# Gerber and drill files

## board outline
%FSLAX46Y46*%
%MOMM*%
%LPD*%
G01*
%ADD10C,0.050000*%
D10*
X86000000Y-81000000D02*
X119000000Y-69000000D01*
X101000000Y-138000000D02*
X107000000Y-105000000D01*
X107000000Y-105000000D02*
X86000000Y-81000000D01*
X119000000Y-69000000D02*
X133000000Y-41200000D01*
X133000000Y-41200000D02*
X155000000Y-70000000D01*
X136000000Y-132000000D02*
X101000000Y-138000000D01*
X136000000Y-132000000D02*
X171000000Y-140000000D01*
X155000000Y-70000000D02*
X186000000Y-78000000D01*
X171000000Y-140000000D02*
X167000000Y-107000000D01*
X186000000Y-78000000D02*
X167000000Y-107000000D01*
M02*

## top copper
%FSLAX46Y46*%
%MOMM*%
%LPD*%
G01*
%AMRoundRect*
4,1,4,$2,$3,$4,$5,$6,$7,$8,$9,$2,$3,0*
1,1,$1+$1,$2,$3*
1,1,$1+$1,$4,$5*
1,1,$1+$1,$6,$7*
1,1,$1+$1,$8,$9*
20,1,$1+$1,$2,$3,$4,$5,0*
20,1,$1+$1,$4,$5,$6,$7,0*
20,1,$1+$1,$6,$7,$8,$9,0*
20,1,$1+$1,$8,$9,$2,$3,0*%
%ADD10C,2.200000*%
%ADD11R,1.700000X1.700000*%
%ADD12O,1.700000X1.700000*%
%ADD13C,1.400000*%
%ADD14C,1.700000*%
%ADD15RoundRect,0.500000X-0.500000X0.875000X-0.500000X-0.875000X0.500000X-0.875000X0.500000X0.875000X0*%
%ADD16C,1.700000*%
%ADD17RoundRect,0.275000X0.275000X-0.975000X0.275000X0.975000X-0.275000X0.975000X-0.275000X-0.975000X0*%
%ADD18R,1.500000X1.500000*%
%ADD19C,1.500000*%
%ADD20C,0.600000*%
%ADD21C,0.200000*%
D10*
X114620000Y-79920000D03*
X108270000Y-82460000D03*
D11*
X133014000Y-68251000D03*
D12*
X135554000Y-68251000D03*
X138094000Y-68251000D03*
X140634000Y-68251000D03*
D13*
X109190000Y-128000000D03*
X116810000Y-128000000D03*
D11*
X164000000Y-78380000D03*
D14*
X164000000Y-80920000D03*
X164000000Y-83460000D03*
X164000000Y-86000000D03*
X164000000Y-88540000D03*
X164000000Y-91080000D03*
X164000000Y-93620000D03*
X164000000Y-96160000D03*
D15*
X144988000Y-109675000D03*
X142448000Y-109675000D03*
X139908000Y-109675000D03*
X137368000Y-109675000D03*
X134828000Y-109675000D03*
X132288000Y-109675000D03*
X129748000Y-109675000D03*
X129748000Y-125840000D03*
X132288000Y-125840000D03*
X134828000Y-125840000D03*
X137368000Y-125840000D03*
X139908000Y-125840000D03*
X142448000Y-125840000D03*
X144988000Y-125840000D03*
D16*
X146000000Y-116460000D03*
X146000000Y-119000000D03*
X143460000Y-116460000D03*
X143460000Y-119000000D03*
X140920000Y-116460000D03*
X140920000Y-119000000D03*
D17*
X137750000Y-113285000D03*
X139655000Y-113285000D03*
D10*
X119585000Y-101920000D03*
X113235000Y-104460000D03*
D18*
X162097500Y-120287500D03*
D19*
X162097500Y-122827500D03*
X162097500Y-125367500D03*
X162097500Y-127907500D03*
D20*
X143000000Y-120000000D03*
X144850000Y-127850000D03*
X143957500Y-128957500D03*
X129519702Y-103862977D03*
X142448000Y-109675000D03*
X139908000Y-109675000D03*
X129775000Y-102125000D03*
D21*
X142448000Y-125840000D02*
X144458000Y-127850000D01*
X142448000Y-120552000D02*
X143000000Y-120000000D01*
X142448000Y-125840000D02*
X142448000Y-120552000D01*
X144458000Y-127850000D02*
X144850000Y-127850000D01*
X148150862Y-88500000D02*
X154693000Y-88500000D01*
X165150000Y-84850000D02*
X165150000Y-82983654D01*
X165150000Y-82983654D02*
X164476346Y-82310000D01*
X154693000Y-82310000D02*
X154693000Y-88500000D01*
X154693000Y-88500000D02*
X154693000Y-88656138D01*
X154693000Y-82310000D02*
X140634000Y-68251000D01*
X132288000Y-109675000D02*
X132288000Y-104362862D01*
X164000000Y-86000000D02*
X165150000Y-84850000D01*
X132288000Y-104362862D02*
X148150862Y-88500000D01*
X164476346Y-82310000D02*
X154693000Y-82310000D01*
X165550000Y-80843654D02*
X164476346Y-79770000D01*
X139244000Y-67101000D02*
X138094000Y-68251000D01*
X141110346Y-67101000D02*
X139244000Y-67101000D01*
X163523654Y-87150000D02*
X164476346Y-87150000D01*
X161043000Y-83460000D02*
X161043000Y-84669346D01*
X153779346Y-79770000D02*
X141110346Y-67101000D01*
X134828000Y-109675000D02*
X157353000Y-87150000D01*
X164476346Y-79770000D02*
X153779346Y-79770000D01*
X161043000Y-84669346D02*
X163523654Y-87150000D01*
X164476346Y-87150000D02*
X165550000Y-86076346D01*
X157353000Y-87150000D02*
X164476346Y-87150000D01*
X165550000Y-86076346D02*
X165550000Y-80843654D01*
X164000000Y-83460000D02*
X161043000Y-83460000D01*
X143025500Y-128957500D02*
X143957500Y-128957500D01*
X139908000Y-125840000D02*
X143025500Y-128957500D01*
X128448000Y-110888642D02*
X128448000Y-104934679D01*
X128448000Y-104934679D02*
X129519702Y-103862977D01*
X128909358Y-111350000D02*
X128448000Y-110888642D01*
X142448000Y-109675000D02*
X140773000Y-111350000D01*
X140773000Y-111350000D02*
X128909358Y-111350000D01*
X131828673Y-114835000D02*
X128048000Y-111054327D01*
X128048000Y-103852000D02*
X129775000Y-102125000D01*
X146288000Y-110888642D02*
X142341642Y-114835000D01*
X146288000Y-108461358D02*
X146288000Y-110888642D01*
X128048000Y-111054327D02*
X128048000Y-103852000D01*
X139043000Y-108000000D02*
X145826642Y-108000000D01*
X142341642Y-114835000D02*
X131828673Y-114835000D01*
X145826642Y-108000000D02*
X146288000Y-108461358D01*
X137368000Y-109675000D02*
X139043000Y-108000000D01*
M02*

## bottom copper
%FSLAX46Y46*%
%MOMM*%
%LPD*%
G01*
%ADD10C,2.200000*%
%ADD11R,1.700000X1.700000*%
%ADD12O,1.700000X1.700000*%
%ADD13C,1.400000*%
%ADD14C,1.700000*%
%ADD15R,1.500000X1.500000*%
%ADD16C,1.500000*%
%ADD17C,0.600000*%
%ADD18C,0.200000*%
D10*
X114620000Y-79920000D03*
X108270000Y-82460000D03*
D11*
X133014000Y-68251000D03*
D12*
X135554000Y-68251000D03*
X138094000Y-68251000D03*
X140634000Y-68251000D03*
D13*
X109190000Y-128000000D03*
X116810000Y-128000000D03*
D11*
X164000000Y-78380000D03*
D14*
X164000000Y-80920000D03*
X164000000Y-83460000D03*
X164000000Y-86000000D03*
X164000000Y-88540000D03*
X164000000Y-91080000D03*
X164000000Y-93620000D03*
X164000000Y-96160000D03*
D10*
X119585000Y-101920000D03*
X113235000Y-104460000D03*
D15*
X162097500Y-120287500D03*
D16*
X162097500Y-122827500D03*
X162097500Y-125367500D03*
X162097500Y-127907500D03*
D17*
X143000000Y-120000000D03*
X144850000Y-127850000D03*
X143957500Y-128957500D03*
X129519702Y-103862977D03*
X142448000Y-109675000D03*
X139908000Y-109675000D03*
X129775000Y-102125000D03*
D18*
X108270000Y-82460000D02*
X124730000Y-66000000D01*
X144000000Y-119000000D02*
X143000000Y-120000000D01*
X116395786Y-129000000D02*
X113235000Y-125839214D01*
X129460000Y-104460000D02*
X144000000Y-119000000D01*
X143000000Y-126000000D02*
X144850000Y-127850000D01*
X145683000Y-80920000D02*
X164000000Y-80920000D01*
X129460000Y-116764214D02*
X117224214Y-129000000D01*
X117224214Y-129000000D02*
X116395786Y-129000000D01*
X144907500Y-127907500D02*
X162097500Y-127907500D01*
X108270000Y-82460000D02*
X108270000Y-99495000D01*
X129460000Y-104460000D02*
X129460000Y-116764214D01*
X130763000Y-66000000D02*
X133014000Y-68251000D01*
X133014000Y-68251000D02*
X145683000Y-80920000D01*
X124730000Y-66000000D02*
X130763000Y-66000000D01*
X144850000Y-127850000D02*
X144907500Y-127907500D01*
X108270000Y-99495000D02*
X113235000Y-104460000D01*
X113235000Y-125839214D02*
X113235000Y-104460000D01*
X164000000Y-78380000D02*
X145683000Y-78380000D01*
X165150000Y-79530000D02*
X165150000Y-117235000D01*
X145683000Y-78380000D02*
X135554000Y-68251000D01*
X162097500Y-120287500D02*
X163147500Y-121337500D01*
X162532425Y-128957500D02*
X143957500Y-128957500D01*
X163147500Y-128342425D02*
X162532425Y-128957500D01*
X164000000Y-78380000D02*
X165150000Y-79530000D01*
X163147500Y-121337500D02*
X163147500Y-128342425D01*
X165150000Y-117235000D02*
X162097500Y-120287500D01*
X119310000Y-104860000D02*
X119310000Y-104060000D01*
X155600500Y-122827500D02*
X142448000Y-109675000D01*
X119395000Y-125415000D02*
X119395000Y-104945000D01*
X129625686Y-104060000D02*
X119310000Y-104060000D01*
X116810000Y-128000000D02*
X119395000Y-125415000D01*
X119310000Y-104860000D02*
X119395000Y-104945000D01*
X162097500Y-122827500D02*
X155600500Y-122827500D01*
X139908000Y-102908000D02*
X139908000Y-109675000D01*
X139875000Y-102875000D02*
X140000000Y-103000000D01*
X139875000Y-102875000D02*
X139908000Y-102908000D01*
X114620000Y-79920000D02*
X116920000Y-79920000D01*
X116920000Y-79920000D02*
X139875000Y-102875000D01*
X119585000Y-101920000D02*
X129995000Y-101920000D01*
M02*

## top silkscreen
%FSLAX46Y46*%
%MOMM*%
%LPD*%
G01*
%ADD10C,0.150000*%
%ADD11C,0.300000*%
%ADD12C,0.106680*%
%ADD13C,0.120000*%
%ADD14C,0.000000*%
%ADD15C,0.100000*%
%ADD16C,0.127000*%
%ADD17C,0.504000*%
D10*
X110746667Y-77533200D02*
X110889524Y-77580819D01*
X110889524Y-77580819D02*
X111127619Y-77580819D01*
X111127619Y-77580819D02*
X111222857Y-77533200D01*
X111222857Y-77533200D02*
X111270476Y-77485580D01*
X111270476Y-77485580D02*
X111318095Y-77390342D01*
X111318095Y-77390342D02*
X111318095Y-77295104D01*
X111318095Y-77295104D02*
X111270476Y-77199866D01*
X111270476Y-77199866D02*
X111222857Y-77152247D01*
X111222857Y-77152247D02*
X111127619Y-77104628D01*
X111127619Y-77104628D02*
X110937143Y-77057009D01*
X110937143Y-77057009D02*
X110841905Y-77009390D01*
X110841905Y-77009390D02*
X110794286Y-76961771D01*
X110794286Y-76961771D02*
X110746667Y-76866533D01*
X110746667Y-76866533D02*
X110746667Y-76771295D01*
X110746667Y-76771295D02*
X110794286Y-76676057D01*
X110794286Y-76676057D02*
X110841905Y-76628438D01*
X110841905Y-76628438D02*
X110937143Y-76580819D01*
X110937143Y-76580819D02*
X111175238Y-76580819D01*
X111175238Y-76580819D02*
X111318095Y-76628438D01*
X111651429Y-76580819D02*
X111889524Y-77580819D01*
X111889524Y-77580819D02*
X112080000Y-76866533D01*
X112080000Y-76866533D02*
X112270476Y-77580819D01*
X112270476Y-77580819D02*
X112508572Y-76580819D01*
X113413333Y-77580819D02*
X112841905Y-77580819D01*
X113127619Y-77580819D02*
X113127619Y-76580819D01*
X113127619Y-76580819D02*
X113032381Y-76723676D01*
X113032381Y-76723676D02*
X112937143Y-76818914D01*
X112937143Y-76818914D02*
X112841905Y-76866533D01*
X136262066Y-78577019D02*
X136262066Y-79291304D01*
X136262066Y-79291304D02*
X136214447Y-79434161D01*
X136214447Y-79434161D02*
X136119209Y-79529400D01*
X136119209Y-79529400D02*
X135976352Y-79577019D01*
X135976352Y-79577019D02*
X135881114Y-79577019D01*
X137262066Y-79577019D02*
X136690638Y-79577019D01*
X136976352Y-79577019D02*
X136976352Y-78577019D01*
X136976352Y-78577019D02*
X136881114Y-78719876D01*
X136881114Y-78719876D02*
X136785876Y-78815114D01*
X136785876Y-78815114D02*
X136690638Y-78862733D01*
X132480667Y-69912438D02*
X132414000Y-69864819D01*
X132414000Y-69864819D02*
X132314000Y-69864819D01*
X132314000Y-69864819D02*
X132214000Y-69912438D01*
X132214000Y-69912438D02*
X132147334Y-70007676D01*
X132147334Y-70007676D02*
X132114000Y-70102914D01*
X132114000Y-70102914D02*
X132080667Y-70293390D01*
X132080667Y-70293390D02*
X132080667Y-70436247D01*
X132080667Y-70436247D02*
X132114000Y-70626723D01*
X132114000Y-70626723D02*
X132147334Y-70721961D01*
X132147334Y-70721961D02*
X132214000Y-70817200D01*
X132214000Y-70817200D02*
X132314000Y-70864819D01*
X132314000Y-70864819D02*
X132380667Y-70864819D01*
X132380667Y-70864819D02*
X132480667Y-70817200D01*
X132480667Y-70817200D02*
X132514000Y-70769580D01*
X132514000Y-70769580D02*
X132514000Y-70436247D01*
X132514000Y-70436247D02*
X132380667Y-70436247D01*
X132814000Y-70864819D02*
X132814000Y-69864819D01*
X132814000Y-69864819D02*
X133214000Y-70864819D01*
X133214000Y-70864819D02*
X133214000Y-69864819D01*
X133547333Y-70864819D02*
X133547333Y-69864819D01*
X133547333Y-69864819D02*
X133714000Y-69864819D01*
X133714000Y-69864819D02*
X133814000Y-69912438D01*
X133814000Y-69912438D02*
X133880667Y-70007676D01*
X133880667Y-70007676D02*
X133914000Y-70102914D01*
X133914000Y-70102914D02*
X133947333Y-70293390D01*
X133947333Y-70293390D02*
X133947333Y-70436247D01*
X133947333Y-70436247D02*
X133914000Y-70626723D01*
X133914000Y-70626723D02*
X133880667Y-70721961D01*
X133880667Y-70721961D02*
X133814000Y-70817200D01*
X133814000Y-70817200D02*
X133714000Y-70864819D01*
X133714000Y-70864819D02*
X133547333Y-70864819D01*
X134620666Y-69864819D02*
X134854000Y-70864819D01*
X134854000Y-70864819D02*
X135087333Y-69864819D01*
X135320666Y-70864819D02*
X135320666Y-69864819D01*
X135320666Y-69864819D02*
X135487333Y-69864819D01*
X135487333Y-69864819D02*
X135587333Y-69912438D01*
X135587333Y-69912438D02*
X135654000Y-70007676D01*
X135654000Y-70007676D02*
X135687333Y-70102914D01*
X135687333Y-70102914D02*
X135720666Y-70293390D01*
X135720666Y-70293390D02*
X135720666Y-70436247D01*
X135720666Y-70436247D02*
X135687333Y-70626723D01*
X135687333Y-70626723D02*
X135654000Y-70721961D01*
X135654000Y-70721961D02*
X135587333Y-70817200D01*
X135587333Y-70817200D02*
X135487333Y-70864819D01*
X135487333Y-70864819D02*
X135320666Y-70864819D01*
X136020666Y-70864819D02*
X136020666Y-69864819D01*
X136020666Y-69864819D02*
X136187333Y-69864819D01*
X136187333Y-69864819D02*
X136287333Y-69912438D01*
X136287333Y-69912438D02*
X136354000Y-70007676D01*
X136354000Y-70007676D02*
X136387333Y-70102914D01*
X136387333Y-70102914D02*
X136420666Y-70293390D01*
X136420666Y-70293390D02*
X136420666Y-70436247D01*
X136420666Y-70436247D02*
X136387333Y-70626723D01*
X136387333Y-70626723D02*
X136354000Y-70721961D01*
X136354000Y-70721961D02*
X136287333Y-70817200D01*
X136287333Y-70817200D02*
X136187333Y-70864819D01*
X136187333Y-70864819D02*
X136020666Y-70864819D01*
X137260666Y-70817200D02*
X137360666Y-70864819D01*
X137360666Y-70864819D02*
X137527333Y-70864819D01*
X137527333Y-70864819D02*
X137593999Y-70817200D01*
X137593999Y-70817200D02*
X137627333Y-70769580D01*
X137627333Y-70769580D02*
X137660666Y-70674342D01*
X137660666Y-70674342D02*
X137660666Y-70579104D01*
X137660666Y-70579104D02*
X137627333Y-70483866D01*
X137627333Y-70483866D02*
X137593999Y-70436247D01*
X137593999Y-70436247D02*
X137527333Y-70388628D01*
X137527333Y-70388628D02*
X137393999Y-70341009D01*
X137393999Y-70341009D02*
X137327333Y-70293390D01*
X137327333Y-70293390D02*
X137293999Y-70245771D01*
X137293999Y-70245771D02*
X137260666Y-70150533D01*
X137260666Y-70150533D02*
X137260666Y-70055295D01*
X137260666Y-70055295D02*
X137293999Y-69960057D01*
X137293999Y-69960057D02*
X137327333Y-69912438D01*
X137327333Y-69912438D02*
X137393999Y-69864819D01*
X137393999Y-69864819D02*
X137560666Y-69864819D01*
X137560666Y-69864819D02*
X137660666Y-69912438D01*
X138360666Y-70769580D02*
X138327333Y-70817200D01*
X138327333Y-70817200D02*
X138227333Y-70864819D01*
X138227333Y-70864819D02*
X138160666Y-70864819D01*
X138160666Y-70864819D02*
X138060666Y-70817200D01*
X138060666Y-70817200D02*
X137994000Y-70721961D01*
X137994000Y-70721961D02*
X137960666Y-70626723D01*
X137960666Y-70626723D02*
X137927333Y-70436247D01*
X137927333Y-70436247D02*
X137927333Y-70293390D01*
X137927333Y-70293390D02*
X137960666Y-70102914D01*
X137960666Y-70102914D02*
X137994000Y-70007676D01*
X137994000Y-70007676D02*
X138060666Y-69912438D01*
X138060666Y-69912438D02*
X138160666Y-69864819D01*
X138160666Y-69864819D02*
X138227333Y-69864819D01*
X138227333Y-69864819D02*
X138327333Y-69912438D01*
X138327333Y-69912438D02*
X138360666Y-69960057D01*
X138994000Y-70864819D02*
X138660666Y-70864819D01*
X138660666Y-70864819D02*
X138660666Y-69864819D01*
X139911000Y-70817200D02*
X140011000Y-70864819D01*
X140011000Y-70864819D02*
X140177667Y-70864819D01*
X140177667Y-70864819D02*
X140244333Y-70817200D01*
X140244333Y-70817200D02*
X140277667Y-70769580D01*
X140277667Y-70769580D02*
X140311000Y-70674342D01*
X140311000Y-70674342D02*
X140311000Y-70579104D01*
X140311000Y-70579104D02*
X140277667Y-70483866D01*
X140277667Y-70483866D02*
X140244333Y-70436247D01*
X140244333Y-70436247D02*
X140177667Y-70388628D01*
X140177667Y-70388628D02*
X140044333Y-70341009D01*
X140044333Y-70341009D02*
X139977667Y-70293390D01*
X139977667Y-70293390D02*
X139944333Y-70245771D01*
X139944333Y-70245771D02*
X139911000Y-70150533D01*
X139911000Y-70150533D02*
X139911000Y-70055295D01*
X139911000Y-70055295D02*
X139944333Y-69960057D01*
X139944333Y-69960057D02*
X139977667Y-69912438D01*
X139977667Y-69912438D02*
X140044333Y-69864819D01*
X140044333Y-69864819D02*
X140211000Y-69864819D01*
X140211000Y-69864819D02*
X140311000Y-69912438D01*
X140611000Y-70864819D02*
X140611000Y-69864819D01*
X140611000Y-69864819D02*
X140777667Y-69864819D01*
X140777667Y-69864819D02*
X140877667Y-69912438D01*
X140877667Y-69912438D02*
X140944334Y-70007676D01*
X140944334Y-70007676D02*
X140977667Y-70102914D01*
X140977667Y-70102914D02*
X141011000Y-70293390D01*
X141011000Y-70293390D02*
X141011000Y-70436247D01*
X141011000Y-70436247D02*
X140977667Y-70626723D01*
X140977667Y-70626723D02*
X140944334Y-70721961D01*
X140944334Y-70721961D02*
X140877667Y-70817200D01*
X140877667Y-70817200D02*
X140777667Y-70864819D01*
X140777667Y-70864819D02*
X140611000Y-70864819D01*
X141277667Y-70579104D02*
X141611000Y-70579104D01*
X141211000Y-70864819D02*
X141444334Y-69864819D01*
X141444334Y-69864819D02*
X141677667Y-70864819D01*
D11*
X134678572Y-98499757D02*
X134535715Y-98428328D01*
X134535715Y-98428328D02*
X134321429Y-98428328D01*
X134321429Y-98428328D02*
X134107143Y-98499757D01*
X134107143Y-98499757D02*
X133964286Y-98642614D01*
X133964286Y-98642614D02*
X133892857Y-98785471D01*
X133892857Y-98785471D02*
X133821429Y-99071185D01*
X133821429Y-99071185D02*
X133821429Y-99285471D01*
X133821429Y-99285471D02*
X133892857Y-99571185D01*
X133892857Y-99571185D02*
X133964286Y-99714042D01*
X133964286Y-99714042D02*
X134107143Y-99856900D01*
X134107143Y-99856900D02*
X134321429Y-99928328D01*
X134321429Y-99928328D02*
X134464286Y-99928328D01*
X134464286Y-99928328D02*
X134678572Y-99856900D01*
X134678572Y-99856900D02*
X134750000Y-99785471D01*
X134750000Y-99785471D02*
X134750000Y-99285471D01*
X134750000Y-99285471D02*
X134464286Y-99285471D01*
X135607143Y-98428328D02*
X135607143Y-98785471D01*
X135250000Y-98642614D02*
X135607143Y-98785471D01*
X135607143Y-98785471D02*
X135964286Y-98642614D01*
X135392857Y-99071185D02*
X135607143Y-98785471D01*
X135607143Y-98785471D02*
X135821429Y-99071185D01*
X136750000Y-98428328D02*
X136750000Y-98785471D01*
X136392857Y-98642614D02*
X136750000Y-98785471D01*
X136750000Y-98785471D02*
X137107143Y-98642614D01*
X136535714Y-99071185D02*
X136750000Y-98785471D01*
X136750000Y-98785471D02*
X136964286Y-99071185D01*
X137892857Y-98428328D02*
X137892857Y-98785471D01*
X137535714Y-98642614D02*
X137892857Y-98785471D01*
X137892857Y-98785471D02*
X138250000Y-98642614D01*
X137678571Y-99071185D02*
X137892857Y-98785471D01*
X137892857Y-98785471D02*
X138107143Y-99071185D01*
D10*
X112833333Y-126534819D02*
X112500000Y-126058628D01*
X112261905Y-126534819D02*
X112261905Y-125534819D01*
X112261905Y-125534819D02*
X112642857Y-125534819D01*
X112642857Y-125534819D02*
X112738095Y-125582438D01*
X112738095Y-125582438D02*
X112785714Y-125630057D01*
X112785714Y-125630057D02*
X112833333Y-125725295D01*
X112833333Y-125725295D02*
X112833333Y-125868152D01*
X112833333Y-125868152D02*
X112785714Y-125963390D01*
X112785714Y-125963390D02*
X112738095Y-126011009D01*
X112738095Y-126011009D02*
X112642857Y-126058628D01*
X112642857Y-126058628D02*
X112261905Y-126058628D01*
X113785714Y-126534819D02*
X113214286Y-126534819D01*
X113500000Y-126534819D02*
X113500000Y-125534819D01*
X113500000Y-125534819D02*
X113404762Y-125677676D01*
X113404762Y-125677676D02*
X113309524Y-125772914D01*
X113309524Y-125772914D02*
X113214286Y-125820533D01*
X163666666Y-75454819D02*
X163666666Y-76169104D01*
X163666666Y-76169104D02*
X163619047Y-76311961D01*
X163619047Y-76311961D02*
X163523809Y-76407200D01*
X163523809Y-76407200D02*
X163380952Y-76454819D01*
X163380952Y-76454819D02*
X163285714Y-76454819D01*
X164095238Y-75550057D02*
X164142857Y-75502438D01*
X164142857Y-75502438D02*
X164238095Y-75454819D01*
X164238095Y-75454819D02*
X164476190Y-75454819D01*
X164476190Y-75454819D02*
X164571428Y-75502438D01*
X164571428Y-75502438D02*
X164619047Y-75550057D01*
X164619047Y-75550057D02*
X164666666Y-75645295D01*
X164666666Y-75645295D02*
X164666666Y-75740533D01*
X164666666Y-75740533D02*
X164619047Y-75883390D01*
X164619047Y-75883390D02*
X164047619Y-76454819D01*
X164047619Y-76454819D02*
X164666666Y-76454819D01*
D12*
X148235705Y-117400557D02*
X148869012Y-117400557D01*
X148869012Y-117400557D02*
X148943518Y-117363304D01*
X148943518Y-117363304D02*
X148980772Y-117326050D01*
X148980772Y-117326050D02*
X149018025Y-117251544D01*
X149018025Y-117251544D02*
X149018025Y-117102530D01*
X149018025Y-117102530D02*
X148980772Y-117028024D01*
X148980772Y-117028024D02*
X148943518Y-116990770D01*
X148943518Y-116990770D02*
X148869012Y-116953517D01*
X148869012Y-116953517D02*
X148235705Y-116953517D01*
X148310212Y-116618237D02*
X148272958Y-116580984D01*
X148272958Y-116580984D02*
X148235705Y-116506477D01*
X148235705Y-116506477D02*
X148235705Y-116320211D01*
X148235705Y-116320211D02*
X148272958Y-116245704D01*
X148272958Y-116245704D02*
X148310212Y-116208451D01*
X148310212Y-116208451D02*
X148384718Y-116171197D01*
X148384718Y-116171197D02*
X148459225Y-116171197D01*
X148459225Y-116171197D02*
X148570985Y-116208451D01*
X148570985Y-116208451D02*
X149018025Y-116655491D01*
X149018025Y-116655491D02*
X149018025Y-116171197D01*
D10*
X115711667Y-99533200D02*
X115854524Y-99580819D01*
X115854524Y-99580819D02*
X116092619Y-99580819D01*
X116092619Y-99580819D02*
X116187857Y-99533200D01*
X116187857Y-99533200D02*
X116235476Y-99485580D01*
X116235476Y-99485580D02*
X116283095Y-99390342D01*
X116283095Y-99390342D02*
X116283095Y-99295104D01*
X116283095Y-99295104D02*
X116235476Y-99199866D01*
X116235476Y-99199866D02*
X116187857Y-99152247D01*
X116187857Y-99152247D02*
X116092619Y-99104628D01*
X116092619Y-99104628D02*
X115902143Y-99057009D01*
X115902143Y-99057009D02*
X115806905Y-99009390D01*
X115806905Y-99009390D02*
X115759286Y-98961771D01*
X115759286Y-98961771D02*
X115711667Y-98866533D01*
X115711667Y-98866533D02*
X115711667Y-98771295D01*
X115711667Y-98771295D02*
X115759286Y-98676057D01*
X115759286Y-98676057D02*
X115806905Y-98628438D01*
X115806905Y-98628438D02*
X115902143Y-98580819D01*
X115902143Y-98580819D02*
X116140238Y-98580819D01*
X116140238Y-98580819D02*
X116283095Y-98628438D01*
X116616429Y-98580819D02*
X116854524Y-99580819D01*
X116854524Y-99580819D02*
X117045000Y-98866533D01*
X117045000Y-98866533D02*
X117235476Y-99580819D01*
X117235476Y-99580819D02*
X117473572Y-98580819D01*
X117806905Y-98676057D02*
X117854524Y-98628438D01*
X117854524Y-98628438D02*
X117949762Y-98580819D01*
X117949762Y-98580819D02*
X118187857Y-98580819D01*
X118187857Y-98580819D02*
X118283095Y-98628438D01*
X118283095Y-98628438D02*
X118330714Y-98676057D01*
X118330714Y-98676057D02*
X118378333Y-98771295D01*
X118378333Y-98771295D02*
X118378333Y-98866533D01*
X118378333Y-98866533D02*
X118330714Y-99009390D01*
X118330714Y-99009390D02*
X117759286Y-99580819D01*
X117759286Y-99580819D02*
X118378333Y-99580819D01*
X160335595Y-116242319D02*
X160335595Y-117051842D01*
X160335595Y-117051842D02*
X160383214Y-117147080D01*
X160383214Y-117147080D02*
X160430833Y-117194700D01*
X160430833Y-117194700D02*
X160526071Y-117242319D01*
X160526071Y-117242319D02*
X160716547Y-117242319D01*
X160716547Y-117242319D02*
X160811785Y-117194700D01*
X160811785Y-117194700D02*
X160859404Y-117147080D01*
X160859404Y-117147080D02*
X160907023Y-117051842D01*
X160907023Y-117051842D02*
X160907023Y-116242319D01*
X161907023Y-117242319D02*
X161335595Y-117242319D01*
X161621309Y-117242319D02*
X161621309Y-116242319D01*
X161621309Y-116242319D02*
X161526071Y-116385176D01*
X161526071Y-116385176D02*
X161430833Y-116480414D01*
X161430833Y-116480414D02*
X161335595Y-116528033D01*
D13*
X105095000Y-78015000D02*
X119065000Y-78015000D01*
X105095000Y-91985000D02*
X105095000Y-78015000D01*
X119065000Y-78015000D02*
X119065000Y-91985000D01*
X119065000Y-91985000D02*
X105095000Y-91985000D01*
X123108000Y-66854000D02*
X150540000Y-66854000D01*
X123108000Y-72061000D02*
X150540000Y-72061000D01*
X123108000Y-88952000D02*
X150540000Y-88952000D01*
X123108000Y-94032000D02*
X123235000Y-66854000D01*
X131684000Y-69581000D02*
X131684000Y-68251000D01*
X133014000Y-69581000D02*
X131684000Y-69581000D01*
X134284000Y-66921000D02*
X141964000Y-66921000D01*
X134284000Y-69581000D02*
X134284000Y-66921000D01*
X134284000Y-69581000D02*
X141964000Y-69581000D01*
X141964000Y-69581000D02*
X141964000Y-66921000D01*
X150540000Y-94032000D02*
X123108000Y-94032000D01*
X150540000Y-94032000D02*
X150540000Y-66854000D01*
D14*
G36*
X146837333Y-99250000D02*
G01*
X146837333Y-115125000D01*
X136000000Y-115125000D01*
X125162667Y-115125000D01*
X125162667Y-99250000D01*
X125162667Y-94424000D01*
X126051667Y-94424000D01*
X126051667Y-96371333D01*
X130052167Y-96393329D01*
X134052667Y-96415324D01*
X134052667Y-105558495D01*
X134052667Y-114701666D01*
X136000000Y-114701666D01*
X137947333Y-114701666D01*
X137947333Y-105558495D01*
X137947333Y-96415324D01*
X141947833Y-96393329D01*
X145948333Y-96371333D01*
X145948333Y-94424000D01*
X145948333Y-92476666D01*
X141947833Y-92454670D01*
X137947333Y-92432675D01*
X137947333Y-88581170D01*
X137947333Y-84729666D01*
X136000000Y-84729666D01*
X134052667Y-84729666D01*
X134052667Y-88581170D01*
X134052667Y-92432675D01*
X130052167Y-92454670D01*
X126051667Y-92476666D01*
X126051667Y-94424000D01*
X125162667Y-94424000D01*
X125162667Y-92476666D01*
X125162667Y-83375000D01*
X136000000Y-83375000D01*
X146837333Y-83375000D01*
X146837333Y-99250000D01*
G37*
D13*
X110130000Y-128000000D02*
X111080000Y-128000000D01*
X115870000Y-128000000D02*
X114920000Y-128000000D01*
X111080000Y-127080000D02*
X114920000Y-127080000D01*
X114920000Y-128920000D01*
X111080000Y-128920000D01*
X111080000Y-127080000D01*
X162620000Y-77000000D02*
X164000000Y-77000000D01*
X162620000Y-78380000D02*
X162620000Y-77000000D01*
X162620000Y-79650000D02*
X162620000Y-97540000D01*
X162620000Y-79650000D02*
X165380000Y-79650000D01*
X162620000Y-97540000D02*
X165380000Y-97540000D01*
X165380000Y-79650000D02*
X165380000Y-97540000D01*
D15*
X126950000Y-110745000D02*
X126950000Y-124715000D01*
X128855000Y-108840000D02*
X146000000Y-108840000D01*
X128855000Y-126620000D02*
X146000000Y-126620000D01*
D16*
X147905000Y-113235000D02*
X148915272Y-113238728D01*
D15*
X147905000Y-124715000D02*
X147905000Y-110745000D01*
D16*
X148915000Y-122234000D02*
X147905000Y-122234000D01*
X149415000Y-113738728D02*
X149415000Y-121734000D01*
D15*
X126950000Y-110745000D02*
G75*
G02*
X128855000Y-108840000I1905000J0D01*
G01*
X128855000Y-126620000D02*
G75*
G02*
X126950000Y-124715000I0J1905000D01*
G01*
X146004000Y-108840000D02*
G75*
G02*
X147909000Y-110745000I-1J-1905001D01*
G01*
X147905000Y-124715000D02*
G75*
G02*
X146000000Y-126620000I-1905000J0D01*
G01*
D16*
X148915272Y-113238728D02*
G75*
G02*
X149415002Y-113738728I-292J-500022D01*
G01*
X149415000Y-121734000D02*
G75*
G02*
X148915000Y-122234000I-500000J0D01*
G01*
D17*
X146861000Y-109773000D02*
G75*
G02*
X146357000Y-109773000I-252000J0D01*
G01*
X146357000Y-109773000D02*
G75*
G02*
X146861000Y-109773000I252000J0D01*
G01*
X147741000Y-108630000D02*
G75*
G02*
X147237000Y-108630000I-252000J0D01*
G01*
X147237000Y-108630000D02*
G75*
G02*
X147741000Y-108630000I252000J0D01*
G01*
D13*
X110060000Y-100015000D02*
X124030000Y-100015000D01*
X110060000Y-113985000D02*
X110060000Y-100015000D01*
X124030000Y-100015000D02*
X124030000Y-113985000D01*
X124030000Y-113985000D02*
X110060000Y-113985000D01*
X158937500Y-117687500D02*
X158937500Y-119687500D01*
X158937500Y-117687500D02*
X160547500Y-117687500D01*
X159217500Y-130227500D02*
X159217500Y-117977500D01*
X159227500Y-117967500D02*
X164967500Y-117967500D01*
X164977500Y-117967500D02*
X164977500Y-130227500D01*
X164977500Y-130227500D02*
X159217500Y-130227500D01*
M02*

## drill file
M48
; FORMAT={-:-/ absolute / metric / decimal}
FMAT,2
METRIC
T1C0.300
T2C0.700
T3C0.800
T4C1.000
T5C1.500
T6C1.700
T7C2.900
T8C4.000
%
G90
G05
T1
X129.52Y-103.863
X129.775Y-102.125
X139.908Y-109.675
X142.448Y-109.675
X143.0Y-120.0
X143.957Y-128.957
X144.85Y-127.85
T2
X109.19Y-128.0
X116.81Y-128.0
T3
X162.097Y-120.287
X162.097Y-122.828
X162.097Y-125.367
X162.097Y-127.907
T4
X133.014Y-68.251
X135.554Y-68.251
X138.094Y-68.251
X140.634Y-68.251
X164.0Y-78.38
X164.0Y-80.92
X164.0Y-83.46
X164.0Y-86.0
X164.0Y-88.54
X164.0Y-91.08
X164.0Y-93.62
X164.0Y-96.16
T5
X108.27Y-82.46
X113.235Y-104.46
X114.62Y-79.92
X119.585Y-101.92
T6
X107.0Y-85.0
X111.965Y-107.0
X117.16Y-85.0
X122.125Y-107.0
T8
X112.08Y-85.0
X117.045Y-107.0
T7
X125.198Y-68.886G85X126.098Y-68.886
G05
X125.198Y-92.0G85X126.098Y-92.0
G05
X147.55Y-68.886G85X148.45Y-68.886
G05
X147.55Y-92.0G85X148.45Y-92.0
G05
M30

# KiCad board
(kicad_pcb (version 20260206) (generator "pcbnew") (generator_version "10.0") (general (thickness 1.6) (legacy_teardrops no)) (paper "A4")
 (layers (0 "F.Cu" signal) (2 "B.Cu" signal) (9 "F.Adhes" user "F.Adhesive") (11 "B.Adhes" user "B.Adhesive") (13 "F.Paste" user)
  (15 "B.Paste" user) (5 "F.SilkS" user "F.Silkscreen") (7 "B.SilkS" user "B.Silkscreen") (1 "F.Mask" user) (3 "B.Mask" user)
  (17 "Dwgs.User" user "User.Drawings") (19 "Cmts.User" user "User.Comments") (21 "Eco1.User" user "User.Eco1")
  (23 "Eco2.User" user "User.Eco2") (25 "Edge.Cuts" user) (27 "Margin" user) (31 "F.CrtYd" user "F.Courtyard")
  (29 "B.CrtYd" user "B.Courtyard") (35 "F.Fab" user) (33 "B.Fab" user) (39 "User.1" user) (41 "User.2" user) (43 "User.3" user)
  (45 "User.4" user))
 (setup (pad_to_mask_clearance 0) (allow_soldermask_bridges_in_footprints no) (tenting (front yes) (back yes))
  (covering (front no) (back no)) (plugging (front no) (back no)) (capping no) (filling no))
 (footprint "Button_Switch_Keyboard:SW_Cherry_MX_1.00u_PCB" (layer "F.Cu") (at 114.62 79.92)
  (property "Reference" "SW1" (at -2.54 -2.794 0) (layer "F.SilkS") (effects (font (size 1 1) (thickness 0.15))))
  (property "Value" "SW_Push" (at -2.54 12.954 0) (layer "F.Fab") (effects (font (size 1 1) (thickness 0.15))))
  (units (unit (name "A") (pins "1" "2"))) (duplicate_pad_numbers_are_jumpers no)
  (fp_line (start -9.525 -1.905) (end 4.445 -1.905) (stroke (width 0.12) (type solid)) (layer "F.SilkS"))
  (fp_line (start -9.525 12.065) (end -9.525 -1.905) (stroke (width 0.12) (type solid)) (layer "F.SilkS"))
  (fp_line (start 4.445 -1.905) (end 4.445 12.065) (stroke (width 0.12) (type solid)) (layer "F.SilkS"))
  (fp_line (start 4.445 12.065) (end -9.525 12.065) (stroke (width 0.12) (type solid)) (layer "F.SilkS"))
  (pad "" np_thru_hole circle (at -7.62 5.08) (size 1.7 1.7) (drill 1.7) (layers "*.Cu" "*.Mask"))
  (pad "" np_thru_hole circle (at -2.54 5.08) (size 4 4) (drill 4) (layers "*.Cu" "*.Mask"))
  (pad "" np_thru_hole circle (at 2.54 5.08) (size 1.7 1.7) (drill 1.7) (layers "*.Cu" "*.Mask"))
  (pad "1" thru_hole circle (at 0 0) (size 2.2 2.2) (drill 1.5) (layers "*.Cu" "*.Mask") (remove_unused_layers no) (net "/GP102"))
  (pad "2" thru_hole circle (at -6.35 2.54) (size 2.2 2.2) (drill 1.5) (layers "*.Cu" "*.Mask") (remove_unused_layers no) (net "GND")))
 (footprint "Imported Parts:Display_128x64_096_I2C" (layer "F.Cu") (at 136.824 68.251)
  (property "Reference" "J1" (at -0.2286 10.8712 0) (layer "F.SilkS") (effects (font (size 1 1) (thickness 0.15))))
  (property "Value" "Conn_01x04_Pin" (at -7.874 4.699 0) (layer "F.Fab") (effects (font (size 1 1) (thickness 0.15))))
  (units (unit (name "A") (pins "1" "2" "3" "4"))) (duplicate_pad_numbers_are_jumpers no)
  (fp_line (start -13.716 -1.397) (end 13.716 -1.397) (stroke (width 0.12) (type solid)) (layer "F.SilkS"))
  (fp_line (start -13.716 3.81) (end 13.716 3.81) (stroke (width 0.12) (type solid)) (layer "F.SilkS"))
  (fp_line (start -13.716 20.701) (end 13.716 20.701) (stroke (width 0.12) (type solid)) (layer "F.SilkS"))
  (fp_line (start -13.716 25.781) (end -13.589 -1.397) (stroke (width 0.12) (type solid)) (layer "F.SilkS"))
  (fp_line (start -5.14 1.33) (end -5.14 0) (stroke (width 0.12) (type solid)) (layer "F.SilkS"))
  (fp_line (start -3.81 1.33) (end -5.14 1.33) (stroke (width 0.12) (type solid)) (layer "F.SilkS"))
  (fp_line (start -2.54 -1.33) (end 5.14 -1.33) (stroke (width 0.12) (type solid)) (layer "F.SilkS"))
  (fp_line (start -2.54 1.33) (end -2.54 -1.33) (stroke (width 0.12) (type solid)) (layer "F.SilkS"))
  (fp_line (start -2.54 1.33) (end 5.14 1.33) (stroke (width 0.12) (type solid)) (layer "F.SilkS"))
  (fp_line (start 5.14 1.33) (end 5.14 -1.33) (stroke (width 0.12) (type solid)) (layer "F.SilkS"))
  (fp_line (start 13.716 25.781) (end -13.716 25.781) (stroke (width 0.12) (type solid)) (layer "F.SilkS"))
  (fp_line (start 13.716 25.781) (end 13.716 -1.397) (stroke (width 0.12) (type solid)) (layer "F.SilkS"))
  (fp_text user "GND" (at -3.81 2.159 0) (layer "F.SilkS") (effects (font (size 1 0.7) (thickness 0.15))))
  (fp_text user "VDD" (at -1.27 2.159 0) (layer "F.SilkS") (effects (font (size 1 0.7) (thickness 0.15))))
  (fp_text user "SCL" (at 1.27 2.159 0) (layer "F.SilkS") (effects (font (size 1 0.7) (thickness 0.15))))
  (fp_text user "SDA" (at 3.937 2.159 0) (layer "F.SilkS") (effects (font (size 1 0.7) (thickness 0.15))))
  (pad "" np_thru_hole oval (at -11.176 0.635) (size 3.8 2.9) (drill oval 3.8 2.9) (layers "*.Cu" "*.Mask"))
  (pad "" np_thru_hole oval (at -11.176 23.749) (size 3.8 2.9) (drill oval 3.8 2.9) (layers "*.Cu" "*.Mask"))
  (pad "" np_thru_hole oval (at 11.176 0.635) (size 3.8 2.9) (drill oval 3.8 2.9) (layers "*.Cu" "*.Mask"))
  (pad "" np_thru_hole oval (at 11.176 23.749) (size 3.8 2.9) (drill oval 3.8 2.9) (layers "*.Cu" "*.Mask"))
  (pad "1" thru_hole rect (at -3.81 0 90) (size 1.7 1.7) (drill 1) (layers "*.Cu" "*.Mask") (remove_unused_layers no) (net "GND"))
  (pad "2" thru_hole oval (at -1.27 0 90) (size 1.7 1.7) (drill 1) (layers "*.Cu" "*.Mask") (remove_unused_layers no) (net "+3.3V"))
  (pad "3" thru_hole oval (at 1.27 0 90) (size 1.7 1.7) (drill 1) (layers "*.Cu" "*.Mask") (remove_unused_layers no) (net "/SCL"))
  (pad "4" thru_hole oval (at 3.81 0 90) (size 1.7 1.7) (drill 1) (layers "*.Cu" "*.Mask") (remove_unused_layers no) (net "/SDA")))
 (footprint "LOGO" (layer "F.Cu") (at 136 99.25)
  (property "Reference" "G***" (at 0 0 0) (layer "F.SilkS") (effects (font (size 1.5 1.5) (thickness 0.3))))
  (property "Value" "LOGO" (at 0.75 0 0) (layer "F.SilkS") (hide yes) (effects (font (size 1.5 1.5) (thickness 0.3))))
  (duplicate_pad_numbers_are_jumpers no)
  (fp_poly
   (pts (xy 10.837333 0) (xy 10.837333 15.875) (xy 0 15.875) (xy -10.837333 15.875) (xy -10.837333 0) (xy -10.837333 -6.773334)
    (xy -9.948333 -6.773334) (xy -9.948333 -4.826) (xy -9.948333 -2.878667) (xy -5.947833 -2.856671) (xy -1.947333 -2.834676)
    (xy -1.947333 6.308495) (xy -1.947333 15.451666) (xy 0 15.451666) (xy 1.947333 15.451666) (xy 1.947333 6.308495) (xy 1.947333 -2.834676)
    (xy 5.947833 -2.856671) (xy 9.948333 -2.878667) (xy 9.948333 -4.826) (xy 9.948333 -6.773334) (xy 5.947833 -6.79533)
    (xy 1.947333 -6.817325) (xy 1.947333 -10.66883) (xy 1.947333 -14.520334) (xy 0 -14.520334) (xy -1.947333 -14.520334)
    (xy -1.947333 -10.66883) (xy -1.947333 -6.817325) (xy -5.947833 -6.79533) (xy -9.948333 -6.773334) (xy -10.837333 -6.773334)
    (xy -10.837333 -15.875) (xy 0 -15.875) (xy 10.837333 -15.875))
   (stroke (width 0) (type solid)) (fill yes) (layer "F.SilkS")))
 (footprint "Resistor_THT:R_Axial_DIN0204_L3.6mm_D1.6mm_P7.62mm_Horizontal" (layer "F.Cu") (at 109.19 128)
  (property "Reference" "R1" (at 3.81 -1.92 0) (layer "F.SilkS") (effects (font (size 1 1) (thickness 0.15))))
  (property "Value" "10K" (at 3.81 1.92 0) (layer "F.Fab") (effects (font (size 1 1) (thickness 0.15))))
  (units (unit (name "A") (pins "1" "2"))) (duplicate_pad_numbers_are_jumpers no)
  (fp_line (start 0.94 0) (end 1.89 0) (stroke (width 0.12) (type solid)) (layer "F.SilkS"))
  (fp_line (start 6.68 0) (end 5.73 0) (stroke (width 0.12) (type solid)) (layer "F.SilkS"))
  (fp_rect (start 1.89 -0.92) (end 5.73 0.92) (stroke (width 0.12) (type solid)) (fill no) (layer "F.SilkS"))
  (pad "1" thru_hole circle (at 0 0) (size 1.4 1.4) (drill 0.7) (layers "*.Cu" "*.Mask") (remove_unused_layers no)
   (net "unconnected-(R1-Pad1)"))
  (pad "2" thru_hole circle (at 7.62 0) (size 1.4 1.4) (drill 0.7) (layers "*.Cu" "*.Mask") (remove_unused_layers no) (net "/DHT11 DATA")))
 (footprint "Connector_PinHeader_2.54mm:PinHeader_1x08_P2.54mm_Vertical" (layer "F.Cu") (at 164 78.38)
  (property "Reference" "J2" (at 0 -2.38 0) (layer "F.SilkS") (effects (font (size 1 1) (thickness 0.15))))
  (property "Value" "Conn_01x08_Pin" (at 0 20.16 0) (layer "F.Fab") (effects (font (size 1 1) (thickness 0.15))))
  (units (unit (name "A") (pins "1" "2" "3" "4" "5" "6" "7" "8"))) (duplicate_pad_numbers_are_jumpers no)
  (fp_line (start -1.38 -1.38) (end 0 -1.38) (stroke (width 0.12) (type solid)) (layer "F.SilkS"))
  (fp_line (start -1.38 0) (end -1.38 -1.38) (stroke (width 0.12) (type solid)) (layer "F.SilkS"))
  (fp_line (start -1.38 1.27) (end -1.38 19.16) (stroke (width 0.12) (type solid)) (layer "F.SilkS"))
  (fp_line (start -1.38 1.27) (end 1.38 1.27) (stroke (width 0.12) (type solid)) (layer "F.SilkS"))
  (fp_line (start -1.38 19.16) (end 1.38 19.16) (stroke (width 0.12) (type solid)) (layer "F.SilkS"))
  (fp_line (start 1.38 1.27) (end 1.38 19.16) (stroke (width 0.12) (type solid)) (layer "F.SilkS"))
  (pad "1" thru_hole rect (at 0 0) (size 1.7 1.7) (drill 1) (layers "*.Cu" "*.Mask") (remove_unused_layers no) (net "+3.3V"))
  (pad "2" thru_hole circle (at 0 2.54) (size 1.7 1.7) (drill 1) (layers "*.Cu" "*.Mask") (remove_unused_layers no) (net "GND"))
  (pad "3" thru_hole circle (at 0 5.08) (size 1.7 1.7) (drill 1) (layers "*.Cu" "*.Mask") (remove_unused_layers no) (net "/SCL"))
  (pad "4" thru_hole circle (at 0 7.62) (size 1.7 1.7) (drill 1) (layers "*.Cu" "*.Mask") (remove_unused_layers no) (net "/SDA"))
  (pad "5" thru_hole circle (at 0 10.16) (size 1.7 1.7) (drill 1) (layers "*.Cu" "*.Mask") (remove_unused_layers no)
   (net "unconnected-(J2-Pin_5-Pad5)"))
  (pad "6" thru_hole circle (at 0 12.7) (size 1.7 1.7) (drill 1) (layers "*.Cu" "*.Mask") (remove_unused_layers no)
   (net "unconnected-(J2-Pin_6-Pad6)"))
  (pad "7" thru_hole circle (at 0 15.24) (size 1.7 1.7) (drill 1) (layers "*.Cu" "*.Mask") (remove_unused_layers no)
   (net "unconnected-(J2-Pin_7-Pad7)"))
  (pad "8" thru_hole circle (at 0 17.78) (size 1.7 1.7) (drill 1) (layers "*.Cu" "*.Mask") (remove_unused_layers no)
   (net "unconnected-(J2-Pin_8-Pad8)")))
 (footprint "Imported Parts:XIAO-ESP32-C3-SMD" (layer "F.Cu") (at 126.868 108.84 -90)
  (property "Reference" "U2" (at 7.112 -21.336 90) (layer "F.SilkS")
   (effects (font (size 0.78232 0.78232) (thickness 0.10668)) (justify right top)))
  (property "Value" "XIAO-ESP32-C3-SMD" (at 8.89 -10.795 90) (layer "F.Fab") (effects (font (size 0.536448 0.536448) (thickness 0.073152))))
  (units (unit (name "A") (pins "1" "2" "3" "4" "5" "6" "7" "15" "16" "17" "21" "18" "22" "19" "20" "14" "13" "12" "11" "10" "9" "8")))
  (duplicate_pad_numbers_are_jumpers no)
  (fp_line (start 1.905 -0.082) (end 15.875 -0.082) (stroke (width 0.1) (type solid)) (layer "F.SilkS"))
  (fp_line (start 0 -1.987) (end 0 -19.132) (stroke (width 0.1) (type solid)) (layer "F.SilkS"))
  (fp_line (start 17.78 -1.987) (end 17.78 -19.132) (stroke (width 0.1) (type solid)) (layer "F.SilkS"))
  (fp_line (start 4.395 -21.037) (end 4.398728 -22.047272) (stroke (width 0.127) (type solid)) (layer "F.SilkS"))
  (fp_line (start 15.875 -21.037) (end 1.905 -21.037) (stroke (width 0.1) (type solid)) (layer "F.SilkS"))
  (fp_line (start 13.394 -22.047) (end 13.394 -21.037) (stroke (width 0.127) (type solid)) (layer "F.SilkS"))
  (fp_line (start 4.898728 -22.547) (end 12.894 -22.547) (stroke (width 0.127) (type solid)) (layer "F.SilkS"))
  (fp_arc (start 1.905 -0.082) (mid 0.557962 -0.639962) (end 0 -1.987) (stroke (width 0.1) (type solid)) (layer "F.SilkS"))
  (fp_arc (start 17.78 -1.987) (mid 17.222038 -0.639962) (end 15.875 -0.082) (stroke (width 0.1) (type solid)) (layer "F.SilkS"))
  (fp_arc (start 0 -19.136) (mid 0.557962 -20.483038) (end 1.905 -21.041) (stroke (width 0.1) (type solid)) (layer "F.SilkS"))
  (fp_arc (start 15.875 -21.037) (mid 17.222038 -20.479038) (end 17.78 -19.132) (stroke (width 0.1) (type solid)) (layer "F.SilkS"))
  (fp_arc (start 4.398728 -22.047272) (mid 4.545272 -22.40064) (end 4.898728 -22.547) (stroke (width 0.127) (type default))
   (layer "F.SilkS"))
  (fp_arc (start 12.894 -22.547) (mid 13.247553 -22.400553) (end 13.394 -22.047) (stroke (width 0.127) (type default)) (layer "F.SilkS"))
  (fp_circle (center 0.933 -19.741) (end 0.933 -19.995) (stroke (width 0.5) (type solid)) (fill yes) (layer "F.SilkS"))
  (fp_circle (center -0.21 -20.621) (end -0.21 -20.875) (stroke (width 0.5) (type solid)) (fill yes) (layer "F.SilkS"))
  (pad "1" smd roundrect (at 0.835 -18.12 270) (size 2.75 2) (layers "F.Cu" "F.Mask" "F.Paste") (roundrect_rratio 0.25)
   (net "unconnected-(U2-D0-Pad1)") (solder_mask_margin 0.0508) (thermal_bridge_angle 45))
  (pad "2" smd roundrect (at 0.835 -15.58 270) (size 2.75 2) (layers "F.Cu" "F.Mask" "F.Paste") (roundrect_rratio 0.25) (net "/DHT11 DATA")
   (solder_mask_margin 0.0508) (thermal_bridge_angle 45))
  (pad "3" smd roundrect (at 0.835 -13.04 270) (size 2.75 2) (layers "F.Cu" "F.Mask" "F.Paste") (roundrect_rratio 0.25) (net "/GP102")
   (solder_mask_margin 0.0508) (thermal_bridge_angle 45))
  (pad "4" smd roundrect (at 0.835 -10.5 270) (size 2.75 2) (layers "F.Cu" "F.Mask" "F.Paste") (roundrect_rratio 0.25) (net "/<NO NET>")
   (solder_mask_margin 0.0508) (thermal_bridge_angle 45))
  (pad "5" smd roundrect (at 0.835 -7.96 270) (size 2.75 2) (layers "F.Cu" "F.Mask" "F.Paste") (roundrect_rratio 0.25) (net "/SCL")
   (solder_mask_margin 0.0508) (thermal_bridge_angle 45))
  (pad "6" smd roundrect (at 0.835 -5.42 270) (size 2.75 2) (layers "F.Cu" "F.Mask" "F.Paste") (roundrect_rratio 0.25) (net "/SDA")
   (solder_mask_margin 0.0508) (thermal_bridge_angle 45))
  (pad "7" smd roundrect (at 0.835 -2.88 270) (size 2.75 2) (layers "F.Cu" "F.Mask" "F.Paste") (roundrect_rratio 0.25)
   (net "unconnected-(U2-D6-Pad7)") (solder_mask_margin 0.0508) (thermal_bridge_angle 45))
  (pad "8" smd roundrect (at 17 -2.88 270) (size 2.75 2) (layers "F.Cu" "F.Mask" "F.Paste") (roundrect_rratio 0.25)
   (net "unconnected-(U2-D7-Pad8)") (solder_mask_margin 0.0508) (thermal_bridge_angle 45))
  (pad "9" smd roundrect (at 17 -5.42 270) (size 2.75 2) (layers "F.Cu" "F.Mask" "F.Paste") (roundrect_rratio 0.25)
   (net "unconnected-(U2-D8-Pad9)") (solder_mask_margin 0.0508) (thermal_bridge_angle 45))
  (pad "10" smd roundrect (at 17 -7.96 270) (size 2.75 2) (layers "F.Cu" "F.Mask" "F.Paste") (roundrect_rratio 0.25)
   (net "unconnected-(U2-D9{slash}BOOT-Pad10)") (solder_mask_margin 0.0508) (thermal_bridge_angle 45))
  (pad "11" smd roundrect (at 17 -10.5 270) (size 2.75 2) (layers "F.Cu" "F.Mask" "F.Paste") (roundrect_rratio 0.25)
   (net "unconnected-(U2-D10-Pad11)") (solder_mask_margin 0.0508) (thermal_bridge_angle 45))
  (pad "12" smd roundrect (at 17 -13.04 270) (size 2.75 2) (layers "F.Cu" "F.Mask" "F.Paste") (roundrect_rratio 0.25) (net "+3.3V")
   (solder_mask_margin 0.0508) (thermal_bridge_angle 45))
  (pad "13" smd roundrect (at 17 -15.58 270) (size 2.75 2) (layers "F.Cu" "F.Mask" "F.Paste") (roundrect_rratio 0.25) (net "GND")
   (solder_mask_margin 0.0508) (thermal_bridge_angle 45))
  (pad "14" smd roundrect (at 17 -18.12 270) (size 2.75 2) (layers "F.Cu" "F.Mask" "F.Paste") (roundrect_rratio 0.25) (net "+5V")
   (solder_mask_margin 0.0508) (thermal_bridge_angle 45))
  (pad "15" smd circle (at 7.62 -19.132 270) (size 1.7 1.7) (layers "F.Cu" "F.Mask" "F.Paste") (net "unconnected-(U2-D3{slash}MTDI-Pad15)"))
  (pad "16" smd circle (at 10.16 -19.132 270) (size 1.7 1.7) (layers "F.Cu" "F.Mask" "F.Paste") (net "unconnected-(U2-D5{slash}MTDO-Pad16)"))
  (pad "17" smd circle (at 7.62 -16.592 270) (size 1.7 1.7) (layers "F.Cu" "F.Mask" "F.Paste") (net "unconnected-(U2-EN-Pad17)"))
  (pad "18" smd circle (at 10.16 -16.592 270) (size 1.7 1.7) (layers "F.Cu" "F.Mask" "F.Paste") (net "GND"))
  (pad "19" smd circle (at 7.62 -14.052 270) (size 1.7 1.7) (layers "F.Cu" "F.Mask" "F.Paste") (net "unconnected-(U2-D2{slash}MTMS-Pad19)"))
  (pad "20" smd circle (at 10.16 -14.052 270) (size 1.7 1.7) (layers "F.Cu" "F.Mask" "F.Paste") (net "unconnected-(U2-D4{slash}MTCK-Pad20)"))
  (pad "21" smd roundrect (at 4.445 -10.882 90) (size 2.5 1.1) (layers "F.Cu" "F.Mask" "F.Paste") (roundrect_rratio 0.25)
   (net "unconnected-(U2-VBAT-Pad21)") (thermal_bridge_angle 45))
  (pad "22" smd roundrect (at 4.445 -12.787 90) (size 2.5 1.1) (layers "F.Cu" "F.Mask" "F.Paste") (roundrect_rratio 0.25)
   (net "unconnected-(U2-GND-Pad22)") (thermal_bridge_angle 45)))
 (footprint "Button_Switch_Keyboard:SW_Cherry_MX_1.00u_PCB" (layer "F.Cu") (at 119.585 101.92)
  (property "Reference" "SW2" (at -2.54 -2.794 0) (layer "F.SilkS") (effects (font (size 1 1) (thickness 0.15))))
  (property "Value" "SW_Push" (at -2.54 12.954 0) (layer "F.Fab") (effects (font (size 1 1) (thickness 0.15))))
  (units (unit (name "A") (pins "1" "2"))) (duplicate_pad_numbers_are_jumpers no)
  (fp_line (start -9.525 -1.905) (end 4.445 -1.905) (stroke (width 0.12) (type solid)) (layer "F.SilkS"))
  (fp_line (start -9.525 12.065) (end -9.525 -1.905) (stroke (width 0.12) (type solid)) (layer "F.SilkS"))
  (fp_line (start 4.445 -1.905) (end 4.445 12.065) (stroke (width 0.12) (type solid)) (layer "F.SilkS"))
  (fp_line (start 4.445 12.065) (end -9.525 12.065) (stroke (width 0.12) (type solid)) (layer "F.SilkS"))
  (pad "" np_thru_hole circle (at -7.62 5.08) (size 1.7 1.7) (drill 1.7) (layers "*.Cu" "*.Mask"))
  (pad "" np_thru_hole circle (at -2.54 5.08) (size 4 4) (drill 4) (layers "*.Cu" "*.Mask"))
  (pad "" np_thru_hole circle (at 2.54 5.08) (size 1.7 1.7) (drill 1.7) (layers "*.Cu" "*.Mask"))
  (pad "1" thru_hole circle (at 0 0) (size 2.2 2.2) (drill 1.5) (layers "*.Cu" "*.Mask") (remove_unused_layers no) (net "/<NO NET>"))
  (pad "2" thru_hole circle (at -6.35 2.54) (size 2.2 2.2) (drill 1.5) (layers "*.Cu" "*.Mask") (remove_unused_layers no) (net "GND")))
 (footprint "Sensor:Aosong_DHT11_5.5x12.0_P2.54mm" (layer "F.Cu") (at 162.0975 120.2875)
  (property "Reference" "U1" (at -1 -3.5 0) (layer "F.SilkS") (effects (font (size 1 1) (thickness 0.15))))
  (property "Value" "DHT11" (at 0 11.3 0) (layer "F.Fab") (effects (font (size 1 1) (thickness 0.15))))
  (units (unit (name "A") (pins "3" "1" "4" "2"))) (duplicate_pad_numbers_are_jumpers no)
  (fp_line (start -3.16 -2.6) (end -3.16 -0.6) (stroke (width 0.12) (type solid)) (layer "F.SilkS"))
  (fp_line (start -3.16 -2.6) (end -1.55 -2.6) (stroke (width 0.12) (type solid)) (layer "F.SilkS"))
  (fp_line (start -2.88 9.94) (end -2.88 -2.31) (stroke (width 0.12) (type solid)) (layer "F.SilkS"))
  (fp_line (start -2.87 -2.32) (end 2.87 -2.32) (stroke (width 0.12) (type solid)) (layer "F.SilkS"))
  (fp_line (start 2.88 -2.32) (end 2.88 9.94) (stroke (width 0.12) (type solid)) (layer "F.SilkS"))
  (fp_line (start 2.88 9.94) (end -2.88 9.94) (stroke (width 0.12) (type solid)) (layer "F.SilkS"))
  (pad "1" thru_hole rect (at 0 0) (size 1.5 1.5) (drill 0.8) (layers "*.Cu" "*.Mask") (remove_unused_layers no) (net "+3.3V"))
  (pad "2" thru_hole circle (at 0 2.54) (size 1.5 1.5) (drill 0.8) (layers "*.Cu" "*.Mask") (remove_unused_layers no) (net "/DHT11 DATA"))
  (pad "3" thru_hole circle (at 0 5.08) (size 1.5 1.5) (drill 0.8) (layers "*.Cu" "*.Mask") (remove_unused_layers no)
   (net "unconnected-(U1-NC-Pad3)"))
  (pad "4" thru_hole circle (at 0 7.62) (size 1.5 1.5) (drill 0.8) (layers "*.Cu" "*.Mask") (remove_unused_layers no) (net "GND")))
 (gr_line (start 86 81) (end 119 69) (stroke (width 0.05) (type default)) (layer "Edge.Cuts"))
 (gr_line (start 101 138) (end 107 105) (stroke (width 0.05) (type default)) (layer "Edge.Cuts"))
 (gr_line (start 107 105) (end 86 81) (stroke (width 0.05) (type default)) (layer "Edge.Cuts"))
 (gr_line (start 119 69) (end 133 41.2) (stroke (width 0.05) (type default)) (layer "Edge.Cuts"))
 (gr_line (start 133 41.2) (end 155 70) (stroke (width 0.05) (type default)) (layer "Edge.Cuts"))
 (gr_line (start 136 132) (end 101 138) (stroke (width 0.05) (type default)) (layer "Edge.Cuts"))
 (gr_line (start 136 132) (end 171 140) (stroke (width 0.05) (type default)) (layer "Edge.Cuts"))
 (gr_line (start 155 70) (end 186 78) (stroke (width 0.05) (type default)) (layer "Edge.Cuts"))
 (gr_line (start 171 140) (end 167 107) (stroke (width 0.05) (type default)) (layer "Edge.Cuts"))
 (gr_line (start 186 78) (end 167 107) (stroke (width 0.05) (type default)) (layer "Edge.Cuts"))
 (segment (start 142.448 125.84) (end 144.458 127.85) (width 0.2) (layer "F.Cu") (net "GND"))
 (segment (start 142.448 120.552) (end 143 120) (width 0.2) (layer "F.Cu") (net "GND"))
 (segment (start 142.448 125.84) (end 142.448 120.552) (width 0.2) (layer "F.Cu") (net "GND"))
 (segment (start 144.458 127.85) (end 144.85 127.85) (width 0.2) (layer "F.Cu") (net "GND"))
 (via (at 143 120) (size 0.6) (drill 0.3) (layers "F.Cu" "B.Cu") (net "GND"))
 (via (at 144.85 127.85) (size 0.6) (drill 0.3) (layers "F.Cu" "B.Cu") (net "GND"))
 (segment (start 108.27 82.46) (end 124.73 66) (width 0.2) (layer "B.Cu") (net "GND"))
 (segment (start 144 119) (end 143 120) (width 0.2) (layer "B.Cu") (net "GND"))
 (segment (start 116.395786 129) (end 113.235 125.839214) (width 0.2) (layer "B.Cu") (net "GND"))
 (segment (start 129.46 104.46) (end 144 119) (width 0.2) (layer "B.Cu") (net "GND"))
 (segment (start 143 126) (end 144.85 127.85) (width 0.2) (layer "B.Cu") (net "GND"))
 (segment (start 145.683 80.92) (end 164 80.92) (width 0.2) (layer "B.Cu") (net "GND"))
 (segment (start 129.46 116.764214) (end 117.224214 129) (width 0.2) (layer "B.Cu") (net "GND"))
 (segment (start 117.224214 129) (end 116.395786 129) (width 0.2) (layer "B.Cu") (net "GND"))
 (segment (start 144.9075 127.9075) (end 162.0975 127.9075) (width 0.2) (layer "B.Cu") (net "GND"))
 (segment (start 108.27 82.46) (end 108.27 99.495) (width 0.2) (layer "B.Cu") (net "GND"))
 (segment (start 129.46 104.46) (end 129.46 116.764214) (width 0.2) (layer "B.Cu") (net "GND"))
 (segment (start 130.763 66) (end 133.014 68.251) (width 0.2) (layer "B.Cu") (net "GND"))
 (segment (start 133.014 68.251) (end 145.683 80.92) (width 0.2) (layer "B.Cu") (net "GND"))
 (segment (start 124.73 66) (end 130.763 66) (width 0.2) (layer "B.Cu") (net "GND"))
 (segment (start 144.85 127.85) (end 144.9075 127.9075) (width 0.2) (layer "B.Cu") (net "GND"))
 (segment (start 108.27 99.495) (end 113.235 104.46) (width 0.2) (layer "B.Cu") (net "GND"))
 (segment (start 113.235 125.839214) (end 113.235 104.46) (width 0.2) (layer "B.Cu") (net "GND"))
 (segment (start 148.150862 88.5) (end 154.693 88.5) (width 0.2) (layer "F.Cu") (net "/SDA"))
 (segment (start 165.15 84.85) (end 165.15 82.983654) (width 0.2) (layer "F.Cu") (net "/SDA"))
 (segment (start 165.15 82.983654) (end 164.476346 82.31) (width 0.2) (layer "F.Cu") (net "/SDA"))
 (segment (start 154.693 82.31) (end 154.693 88.5) (width 0.2) (layer "F.Cu") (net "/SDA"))
 (segment (start 154.693 88.5) (end 154.693 88.656138) (width 0.2) (layer "F.Cu") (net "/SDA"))
 (segment (start 154.693 82.31) (end 140.634 68.251) (width 0.2) (layer "F.Cu") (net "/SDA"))
 (segment (start 132.288 109.675) (end 132.288 104.362862) (width 0.2) (layer "F.Cu") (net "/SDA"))
 (segment (start 164 86) (end 165.15 84.85) (width 0.2) (layer "F.Cu") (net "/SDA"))
 (segment (start 132.288 104.362862) (end 148.150862 88.5) (width 0.2) (layer "F.Cu") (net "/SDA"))
 (segment (start 164.476346 82.31) (end 154.693 82.31) (width 0.2) (layer "F.Cu") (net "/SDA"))
 (segment (start 165.55 80.843654) (end 164.476346 79.77) (width 0.2) (layer "F.Cu") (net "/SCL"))
 (segment (start 139.244 67.101) (end 138.094 68.251) (width 0.2) (layer "F.Cu") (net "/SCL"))
 (segment (start 141.110346 67.101) (end 139.244 67.101) (width 0.2) (layer "F.Cu") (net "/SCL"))
 (segment (start 163.523654 87.15) (end 164.476346 87.15) (width 0.2) (layer "F.Cu") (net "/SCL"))
 (segment (start 161.043 83.46) (end 161.043 84.669346) (width 0.2) (layer "F.Cu") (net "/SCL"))
 (segment (start 153.779346 79.77) (end 141.110346 67.101) (width 0.2) (layer "F.Cu") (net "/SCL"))
 (segment (start 134.828 109.675) (end 157.353 87.15) (width 0.2) (layer "F.Cu") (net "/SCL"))
 (segment (start 164.476346 79.77) (end 153.779346 79.77) (width 0.2) (layer "F.Cu") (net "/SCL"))
 (segment (start 161.043 84.669346) (end 163.523654 87.15) (width 0.2) (layer "F.Cu") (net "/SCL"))
 (segment (start 164.476346 87.15) (end 165.55 86.076346) (width 0.2) (layer "F.Cu") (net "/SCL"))
 (segment (start 157.353 87.15) (end 164.476346 87.15) (width 0.2) (layer "F.Cu") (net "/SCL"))
 (segment (start 165.55 86.076346) (end 165.55 80.843654) (width 0.2) (layer "F.Cu") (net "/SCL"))
 (segment (start 164 83.46) (end 161.043 83.46) (width 0.2) (layer "F.Cu") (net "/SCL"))
 (segment (start 143.0255 128.9575) (end 143.9575 128.9575) (width 0.2) (layer "F.Cu") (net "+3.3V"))
 (segment (start 139.908 125.84) (end 143.0255 128.9575) (width 0.2) (layer "F.Cu") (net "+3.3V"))
 (via (at 143.9575 128.9575) (size 0.6) (drill 0.3) (layers "F.Cu" "B.Cu") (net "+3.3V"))
 (segment (start 164 78.38) (end 145.683 78.38) (width 0.2) (layer "B.Cu") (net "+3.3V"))
 (segment (start 165.15 79.53) (end 165.15 117.235) (width 0.2) (layer "B.Cu") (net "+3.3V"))
 (segment (start 145.683 78.38) (end 135.554 68.251) (width 0.2) (layer "B.Cu") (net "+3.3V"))
 (segment (start 162.0975 120.2875) (end 163.1475 121.3375) (width 0.2) (layer "B.Cu") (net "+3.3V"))
 (segment (start 162.532425 128.9575) (end 143.9575 128.9575) (width 0.2) (layer "B.Cu") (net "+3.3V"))
 (segment (start 163.1475 128.342425) (end 162.532425 128.9575) (width 0.2) (layer "B.Cu") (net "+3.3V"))
 (segment (start 164 78.38) (end 165.15 79.53) (width 0.2) (layer "B.Cu") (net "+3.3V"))
 (segment (start 163.1475 121.3375) (end 163.1475 128.342425) (width 0.2) (layer "B.Cu") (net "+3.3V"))
 (segment (start 165.15 117.235) (end 162.0975 120.2875) (width 0.2) (layer "B.Cu") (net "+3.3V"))
 (segment (start 128.448 110.888642) (end 128.448 104.934679) (width 0.2) (layer "F.Cu") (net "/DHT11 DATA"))
 (segment (start 128.448 104.934679) (end 129.519702 103.862977) (width 0.2) (layer "F.Cu") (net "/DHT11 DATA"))
 (segment (start 128.909358 111.35) (end 128.448 110.888642) (width 0.2) (layer "F.Cu") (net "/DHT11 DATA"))
 (segment (start 142.448 109.675) (end 140.773 111.35) (width 0.2) (layer "F.Cu") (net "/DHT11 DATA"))
 (segment (start 140.773 111.35) (end 128.909358 111.35) (width 0.2) (layer "F.Cu") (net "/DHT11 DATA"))
 (via (at 129.519702 103.862977) (size 0.6) (drill 0.3) (layers "F.Cu" "B.Cu") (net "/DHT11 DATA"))
 (via (at 142.448 109.675) (size 0.6) (drill 0.3) (layers "F.Cu" "B.Cu") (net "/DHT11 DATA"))
 (segment (start 119.31 104.86) (end 119.31 104.06) (width 0.2) (layer "B.Cu") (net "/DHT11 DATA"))
 (segment (start 155.6005 122.8275) (end 142.448 109.675) (width 0.2) (layer "B.Cu") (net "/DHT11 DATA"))
 (segment (start 119.395 125.415) (end 119.395 104.945) (width 0.2) (layer "B.Cu") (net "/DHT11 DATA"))
 (segment (start 129.625686 104.06) (end 119.31 104.06) (width 0.2) (layer "B.Cu") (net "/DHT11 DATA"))
 (segment (start 116.81 128) (end 119.395 125.415) (width 0.2) (layer "B.Cu") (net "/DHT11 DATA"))
 (segment (start 119.31 104.86) (end 119.395 104.945) (width 0.2) (layer "B.Cu") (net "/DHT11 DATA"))
 (segment (start 162.0975 122.8275) (end 155.6005 122.8275) (width 0.2) (layer "B.Cu") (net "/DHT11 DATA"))
 (via (at 139.908 109.675) (size 0.6) (drill 0.3) (layers "F.Cu" "B.Cu") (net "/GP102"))
 (segment (start 139.908 102.908) (end 139.908 109.675) (width 0.2) (layer "B.Cu") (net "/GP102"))
 (segment (start 139.875 102.875) (end 140 103) (width 0.2) (layer "B.Cu") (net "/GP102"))
 (segment (start 139.875 102.875) (end 139.908 102.908) (width 0.2) (layer "B.Cu") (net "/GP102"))
 (segment (start 114.62 79.92) (end 116.92 79.92) (width 0.2) (layer "B.Cu") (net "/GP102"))
 (segment (start 116.92 79.92) (end 139.875 102.875) (width 0.2) (layer "B.Cu") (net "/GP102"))
 (segment (start 131.828673 114.835) (end 128.048 111.054327) (width 0.2) (layer "F.Cu") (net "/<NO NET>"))
 (segment (start 128.048 103.852) (end 129.775 102.125) (width 0.2) (layer "F.Cu") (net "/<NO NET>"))
 (segment (start 146.288 110.888642) (end 142.341642 114.835) (width 0.2) (layer "F.Cu") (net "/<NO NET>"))
 (segment (start 146.288 108.461358) (end 146.288 110.888642) (width 0.2) (layer "F.Cu") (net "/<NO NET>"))
 (segment (start 128.048 111.054327) (end 128.048 103.852) (width 0.2) (layer "F.Cu") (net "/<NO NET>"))
 (segment (start 139.043 108) (end 145.826642 108) (width 0.2) (layer "F.Cu") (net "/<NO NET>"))
 (segment (start 142.341642 114.835) (end 131.828673 114.835) (width 0.2) (layer "F.Cu") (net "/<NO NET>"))
 (segment (start 145.826642 108) (end 146.288 108.461358) (width 0.2) (layer "F.Cu") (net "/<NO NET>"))
 (segment (start 137.368 109.675) (end 139.043 108) (width 0.2) (layer "F.Cu") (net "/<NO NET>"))
 (via (at 129.775 102.125) (size 0.6) (drill 0.3) (layers "F.Cu" "B.Cu") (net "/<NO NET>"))
 (segment (start 119.585 101.92) (end 129.995 101.92) (width 0.2) (layer "B.Cu") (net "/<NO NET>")))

